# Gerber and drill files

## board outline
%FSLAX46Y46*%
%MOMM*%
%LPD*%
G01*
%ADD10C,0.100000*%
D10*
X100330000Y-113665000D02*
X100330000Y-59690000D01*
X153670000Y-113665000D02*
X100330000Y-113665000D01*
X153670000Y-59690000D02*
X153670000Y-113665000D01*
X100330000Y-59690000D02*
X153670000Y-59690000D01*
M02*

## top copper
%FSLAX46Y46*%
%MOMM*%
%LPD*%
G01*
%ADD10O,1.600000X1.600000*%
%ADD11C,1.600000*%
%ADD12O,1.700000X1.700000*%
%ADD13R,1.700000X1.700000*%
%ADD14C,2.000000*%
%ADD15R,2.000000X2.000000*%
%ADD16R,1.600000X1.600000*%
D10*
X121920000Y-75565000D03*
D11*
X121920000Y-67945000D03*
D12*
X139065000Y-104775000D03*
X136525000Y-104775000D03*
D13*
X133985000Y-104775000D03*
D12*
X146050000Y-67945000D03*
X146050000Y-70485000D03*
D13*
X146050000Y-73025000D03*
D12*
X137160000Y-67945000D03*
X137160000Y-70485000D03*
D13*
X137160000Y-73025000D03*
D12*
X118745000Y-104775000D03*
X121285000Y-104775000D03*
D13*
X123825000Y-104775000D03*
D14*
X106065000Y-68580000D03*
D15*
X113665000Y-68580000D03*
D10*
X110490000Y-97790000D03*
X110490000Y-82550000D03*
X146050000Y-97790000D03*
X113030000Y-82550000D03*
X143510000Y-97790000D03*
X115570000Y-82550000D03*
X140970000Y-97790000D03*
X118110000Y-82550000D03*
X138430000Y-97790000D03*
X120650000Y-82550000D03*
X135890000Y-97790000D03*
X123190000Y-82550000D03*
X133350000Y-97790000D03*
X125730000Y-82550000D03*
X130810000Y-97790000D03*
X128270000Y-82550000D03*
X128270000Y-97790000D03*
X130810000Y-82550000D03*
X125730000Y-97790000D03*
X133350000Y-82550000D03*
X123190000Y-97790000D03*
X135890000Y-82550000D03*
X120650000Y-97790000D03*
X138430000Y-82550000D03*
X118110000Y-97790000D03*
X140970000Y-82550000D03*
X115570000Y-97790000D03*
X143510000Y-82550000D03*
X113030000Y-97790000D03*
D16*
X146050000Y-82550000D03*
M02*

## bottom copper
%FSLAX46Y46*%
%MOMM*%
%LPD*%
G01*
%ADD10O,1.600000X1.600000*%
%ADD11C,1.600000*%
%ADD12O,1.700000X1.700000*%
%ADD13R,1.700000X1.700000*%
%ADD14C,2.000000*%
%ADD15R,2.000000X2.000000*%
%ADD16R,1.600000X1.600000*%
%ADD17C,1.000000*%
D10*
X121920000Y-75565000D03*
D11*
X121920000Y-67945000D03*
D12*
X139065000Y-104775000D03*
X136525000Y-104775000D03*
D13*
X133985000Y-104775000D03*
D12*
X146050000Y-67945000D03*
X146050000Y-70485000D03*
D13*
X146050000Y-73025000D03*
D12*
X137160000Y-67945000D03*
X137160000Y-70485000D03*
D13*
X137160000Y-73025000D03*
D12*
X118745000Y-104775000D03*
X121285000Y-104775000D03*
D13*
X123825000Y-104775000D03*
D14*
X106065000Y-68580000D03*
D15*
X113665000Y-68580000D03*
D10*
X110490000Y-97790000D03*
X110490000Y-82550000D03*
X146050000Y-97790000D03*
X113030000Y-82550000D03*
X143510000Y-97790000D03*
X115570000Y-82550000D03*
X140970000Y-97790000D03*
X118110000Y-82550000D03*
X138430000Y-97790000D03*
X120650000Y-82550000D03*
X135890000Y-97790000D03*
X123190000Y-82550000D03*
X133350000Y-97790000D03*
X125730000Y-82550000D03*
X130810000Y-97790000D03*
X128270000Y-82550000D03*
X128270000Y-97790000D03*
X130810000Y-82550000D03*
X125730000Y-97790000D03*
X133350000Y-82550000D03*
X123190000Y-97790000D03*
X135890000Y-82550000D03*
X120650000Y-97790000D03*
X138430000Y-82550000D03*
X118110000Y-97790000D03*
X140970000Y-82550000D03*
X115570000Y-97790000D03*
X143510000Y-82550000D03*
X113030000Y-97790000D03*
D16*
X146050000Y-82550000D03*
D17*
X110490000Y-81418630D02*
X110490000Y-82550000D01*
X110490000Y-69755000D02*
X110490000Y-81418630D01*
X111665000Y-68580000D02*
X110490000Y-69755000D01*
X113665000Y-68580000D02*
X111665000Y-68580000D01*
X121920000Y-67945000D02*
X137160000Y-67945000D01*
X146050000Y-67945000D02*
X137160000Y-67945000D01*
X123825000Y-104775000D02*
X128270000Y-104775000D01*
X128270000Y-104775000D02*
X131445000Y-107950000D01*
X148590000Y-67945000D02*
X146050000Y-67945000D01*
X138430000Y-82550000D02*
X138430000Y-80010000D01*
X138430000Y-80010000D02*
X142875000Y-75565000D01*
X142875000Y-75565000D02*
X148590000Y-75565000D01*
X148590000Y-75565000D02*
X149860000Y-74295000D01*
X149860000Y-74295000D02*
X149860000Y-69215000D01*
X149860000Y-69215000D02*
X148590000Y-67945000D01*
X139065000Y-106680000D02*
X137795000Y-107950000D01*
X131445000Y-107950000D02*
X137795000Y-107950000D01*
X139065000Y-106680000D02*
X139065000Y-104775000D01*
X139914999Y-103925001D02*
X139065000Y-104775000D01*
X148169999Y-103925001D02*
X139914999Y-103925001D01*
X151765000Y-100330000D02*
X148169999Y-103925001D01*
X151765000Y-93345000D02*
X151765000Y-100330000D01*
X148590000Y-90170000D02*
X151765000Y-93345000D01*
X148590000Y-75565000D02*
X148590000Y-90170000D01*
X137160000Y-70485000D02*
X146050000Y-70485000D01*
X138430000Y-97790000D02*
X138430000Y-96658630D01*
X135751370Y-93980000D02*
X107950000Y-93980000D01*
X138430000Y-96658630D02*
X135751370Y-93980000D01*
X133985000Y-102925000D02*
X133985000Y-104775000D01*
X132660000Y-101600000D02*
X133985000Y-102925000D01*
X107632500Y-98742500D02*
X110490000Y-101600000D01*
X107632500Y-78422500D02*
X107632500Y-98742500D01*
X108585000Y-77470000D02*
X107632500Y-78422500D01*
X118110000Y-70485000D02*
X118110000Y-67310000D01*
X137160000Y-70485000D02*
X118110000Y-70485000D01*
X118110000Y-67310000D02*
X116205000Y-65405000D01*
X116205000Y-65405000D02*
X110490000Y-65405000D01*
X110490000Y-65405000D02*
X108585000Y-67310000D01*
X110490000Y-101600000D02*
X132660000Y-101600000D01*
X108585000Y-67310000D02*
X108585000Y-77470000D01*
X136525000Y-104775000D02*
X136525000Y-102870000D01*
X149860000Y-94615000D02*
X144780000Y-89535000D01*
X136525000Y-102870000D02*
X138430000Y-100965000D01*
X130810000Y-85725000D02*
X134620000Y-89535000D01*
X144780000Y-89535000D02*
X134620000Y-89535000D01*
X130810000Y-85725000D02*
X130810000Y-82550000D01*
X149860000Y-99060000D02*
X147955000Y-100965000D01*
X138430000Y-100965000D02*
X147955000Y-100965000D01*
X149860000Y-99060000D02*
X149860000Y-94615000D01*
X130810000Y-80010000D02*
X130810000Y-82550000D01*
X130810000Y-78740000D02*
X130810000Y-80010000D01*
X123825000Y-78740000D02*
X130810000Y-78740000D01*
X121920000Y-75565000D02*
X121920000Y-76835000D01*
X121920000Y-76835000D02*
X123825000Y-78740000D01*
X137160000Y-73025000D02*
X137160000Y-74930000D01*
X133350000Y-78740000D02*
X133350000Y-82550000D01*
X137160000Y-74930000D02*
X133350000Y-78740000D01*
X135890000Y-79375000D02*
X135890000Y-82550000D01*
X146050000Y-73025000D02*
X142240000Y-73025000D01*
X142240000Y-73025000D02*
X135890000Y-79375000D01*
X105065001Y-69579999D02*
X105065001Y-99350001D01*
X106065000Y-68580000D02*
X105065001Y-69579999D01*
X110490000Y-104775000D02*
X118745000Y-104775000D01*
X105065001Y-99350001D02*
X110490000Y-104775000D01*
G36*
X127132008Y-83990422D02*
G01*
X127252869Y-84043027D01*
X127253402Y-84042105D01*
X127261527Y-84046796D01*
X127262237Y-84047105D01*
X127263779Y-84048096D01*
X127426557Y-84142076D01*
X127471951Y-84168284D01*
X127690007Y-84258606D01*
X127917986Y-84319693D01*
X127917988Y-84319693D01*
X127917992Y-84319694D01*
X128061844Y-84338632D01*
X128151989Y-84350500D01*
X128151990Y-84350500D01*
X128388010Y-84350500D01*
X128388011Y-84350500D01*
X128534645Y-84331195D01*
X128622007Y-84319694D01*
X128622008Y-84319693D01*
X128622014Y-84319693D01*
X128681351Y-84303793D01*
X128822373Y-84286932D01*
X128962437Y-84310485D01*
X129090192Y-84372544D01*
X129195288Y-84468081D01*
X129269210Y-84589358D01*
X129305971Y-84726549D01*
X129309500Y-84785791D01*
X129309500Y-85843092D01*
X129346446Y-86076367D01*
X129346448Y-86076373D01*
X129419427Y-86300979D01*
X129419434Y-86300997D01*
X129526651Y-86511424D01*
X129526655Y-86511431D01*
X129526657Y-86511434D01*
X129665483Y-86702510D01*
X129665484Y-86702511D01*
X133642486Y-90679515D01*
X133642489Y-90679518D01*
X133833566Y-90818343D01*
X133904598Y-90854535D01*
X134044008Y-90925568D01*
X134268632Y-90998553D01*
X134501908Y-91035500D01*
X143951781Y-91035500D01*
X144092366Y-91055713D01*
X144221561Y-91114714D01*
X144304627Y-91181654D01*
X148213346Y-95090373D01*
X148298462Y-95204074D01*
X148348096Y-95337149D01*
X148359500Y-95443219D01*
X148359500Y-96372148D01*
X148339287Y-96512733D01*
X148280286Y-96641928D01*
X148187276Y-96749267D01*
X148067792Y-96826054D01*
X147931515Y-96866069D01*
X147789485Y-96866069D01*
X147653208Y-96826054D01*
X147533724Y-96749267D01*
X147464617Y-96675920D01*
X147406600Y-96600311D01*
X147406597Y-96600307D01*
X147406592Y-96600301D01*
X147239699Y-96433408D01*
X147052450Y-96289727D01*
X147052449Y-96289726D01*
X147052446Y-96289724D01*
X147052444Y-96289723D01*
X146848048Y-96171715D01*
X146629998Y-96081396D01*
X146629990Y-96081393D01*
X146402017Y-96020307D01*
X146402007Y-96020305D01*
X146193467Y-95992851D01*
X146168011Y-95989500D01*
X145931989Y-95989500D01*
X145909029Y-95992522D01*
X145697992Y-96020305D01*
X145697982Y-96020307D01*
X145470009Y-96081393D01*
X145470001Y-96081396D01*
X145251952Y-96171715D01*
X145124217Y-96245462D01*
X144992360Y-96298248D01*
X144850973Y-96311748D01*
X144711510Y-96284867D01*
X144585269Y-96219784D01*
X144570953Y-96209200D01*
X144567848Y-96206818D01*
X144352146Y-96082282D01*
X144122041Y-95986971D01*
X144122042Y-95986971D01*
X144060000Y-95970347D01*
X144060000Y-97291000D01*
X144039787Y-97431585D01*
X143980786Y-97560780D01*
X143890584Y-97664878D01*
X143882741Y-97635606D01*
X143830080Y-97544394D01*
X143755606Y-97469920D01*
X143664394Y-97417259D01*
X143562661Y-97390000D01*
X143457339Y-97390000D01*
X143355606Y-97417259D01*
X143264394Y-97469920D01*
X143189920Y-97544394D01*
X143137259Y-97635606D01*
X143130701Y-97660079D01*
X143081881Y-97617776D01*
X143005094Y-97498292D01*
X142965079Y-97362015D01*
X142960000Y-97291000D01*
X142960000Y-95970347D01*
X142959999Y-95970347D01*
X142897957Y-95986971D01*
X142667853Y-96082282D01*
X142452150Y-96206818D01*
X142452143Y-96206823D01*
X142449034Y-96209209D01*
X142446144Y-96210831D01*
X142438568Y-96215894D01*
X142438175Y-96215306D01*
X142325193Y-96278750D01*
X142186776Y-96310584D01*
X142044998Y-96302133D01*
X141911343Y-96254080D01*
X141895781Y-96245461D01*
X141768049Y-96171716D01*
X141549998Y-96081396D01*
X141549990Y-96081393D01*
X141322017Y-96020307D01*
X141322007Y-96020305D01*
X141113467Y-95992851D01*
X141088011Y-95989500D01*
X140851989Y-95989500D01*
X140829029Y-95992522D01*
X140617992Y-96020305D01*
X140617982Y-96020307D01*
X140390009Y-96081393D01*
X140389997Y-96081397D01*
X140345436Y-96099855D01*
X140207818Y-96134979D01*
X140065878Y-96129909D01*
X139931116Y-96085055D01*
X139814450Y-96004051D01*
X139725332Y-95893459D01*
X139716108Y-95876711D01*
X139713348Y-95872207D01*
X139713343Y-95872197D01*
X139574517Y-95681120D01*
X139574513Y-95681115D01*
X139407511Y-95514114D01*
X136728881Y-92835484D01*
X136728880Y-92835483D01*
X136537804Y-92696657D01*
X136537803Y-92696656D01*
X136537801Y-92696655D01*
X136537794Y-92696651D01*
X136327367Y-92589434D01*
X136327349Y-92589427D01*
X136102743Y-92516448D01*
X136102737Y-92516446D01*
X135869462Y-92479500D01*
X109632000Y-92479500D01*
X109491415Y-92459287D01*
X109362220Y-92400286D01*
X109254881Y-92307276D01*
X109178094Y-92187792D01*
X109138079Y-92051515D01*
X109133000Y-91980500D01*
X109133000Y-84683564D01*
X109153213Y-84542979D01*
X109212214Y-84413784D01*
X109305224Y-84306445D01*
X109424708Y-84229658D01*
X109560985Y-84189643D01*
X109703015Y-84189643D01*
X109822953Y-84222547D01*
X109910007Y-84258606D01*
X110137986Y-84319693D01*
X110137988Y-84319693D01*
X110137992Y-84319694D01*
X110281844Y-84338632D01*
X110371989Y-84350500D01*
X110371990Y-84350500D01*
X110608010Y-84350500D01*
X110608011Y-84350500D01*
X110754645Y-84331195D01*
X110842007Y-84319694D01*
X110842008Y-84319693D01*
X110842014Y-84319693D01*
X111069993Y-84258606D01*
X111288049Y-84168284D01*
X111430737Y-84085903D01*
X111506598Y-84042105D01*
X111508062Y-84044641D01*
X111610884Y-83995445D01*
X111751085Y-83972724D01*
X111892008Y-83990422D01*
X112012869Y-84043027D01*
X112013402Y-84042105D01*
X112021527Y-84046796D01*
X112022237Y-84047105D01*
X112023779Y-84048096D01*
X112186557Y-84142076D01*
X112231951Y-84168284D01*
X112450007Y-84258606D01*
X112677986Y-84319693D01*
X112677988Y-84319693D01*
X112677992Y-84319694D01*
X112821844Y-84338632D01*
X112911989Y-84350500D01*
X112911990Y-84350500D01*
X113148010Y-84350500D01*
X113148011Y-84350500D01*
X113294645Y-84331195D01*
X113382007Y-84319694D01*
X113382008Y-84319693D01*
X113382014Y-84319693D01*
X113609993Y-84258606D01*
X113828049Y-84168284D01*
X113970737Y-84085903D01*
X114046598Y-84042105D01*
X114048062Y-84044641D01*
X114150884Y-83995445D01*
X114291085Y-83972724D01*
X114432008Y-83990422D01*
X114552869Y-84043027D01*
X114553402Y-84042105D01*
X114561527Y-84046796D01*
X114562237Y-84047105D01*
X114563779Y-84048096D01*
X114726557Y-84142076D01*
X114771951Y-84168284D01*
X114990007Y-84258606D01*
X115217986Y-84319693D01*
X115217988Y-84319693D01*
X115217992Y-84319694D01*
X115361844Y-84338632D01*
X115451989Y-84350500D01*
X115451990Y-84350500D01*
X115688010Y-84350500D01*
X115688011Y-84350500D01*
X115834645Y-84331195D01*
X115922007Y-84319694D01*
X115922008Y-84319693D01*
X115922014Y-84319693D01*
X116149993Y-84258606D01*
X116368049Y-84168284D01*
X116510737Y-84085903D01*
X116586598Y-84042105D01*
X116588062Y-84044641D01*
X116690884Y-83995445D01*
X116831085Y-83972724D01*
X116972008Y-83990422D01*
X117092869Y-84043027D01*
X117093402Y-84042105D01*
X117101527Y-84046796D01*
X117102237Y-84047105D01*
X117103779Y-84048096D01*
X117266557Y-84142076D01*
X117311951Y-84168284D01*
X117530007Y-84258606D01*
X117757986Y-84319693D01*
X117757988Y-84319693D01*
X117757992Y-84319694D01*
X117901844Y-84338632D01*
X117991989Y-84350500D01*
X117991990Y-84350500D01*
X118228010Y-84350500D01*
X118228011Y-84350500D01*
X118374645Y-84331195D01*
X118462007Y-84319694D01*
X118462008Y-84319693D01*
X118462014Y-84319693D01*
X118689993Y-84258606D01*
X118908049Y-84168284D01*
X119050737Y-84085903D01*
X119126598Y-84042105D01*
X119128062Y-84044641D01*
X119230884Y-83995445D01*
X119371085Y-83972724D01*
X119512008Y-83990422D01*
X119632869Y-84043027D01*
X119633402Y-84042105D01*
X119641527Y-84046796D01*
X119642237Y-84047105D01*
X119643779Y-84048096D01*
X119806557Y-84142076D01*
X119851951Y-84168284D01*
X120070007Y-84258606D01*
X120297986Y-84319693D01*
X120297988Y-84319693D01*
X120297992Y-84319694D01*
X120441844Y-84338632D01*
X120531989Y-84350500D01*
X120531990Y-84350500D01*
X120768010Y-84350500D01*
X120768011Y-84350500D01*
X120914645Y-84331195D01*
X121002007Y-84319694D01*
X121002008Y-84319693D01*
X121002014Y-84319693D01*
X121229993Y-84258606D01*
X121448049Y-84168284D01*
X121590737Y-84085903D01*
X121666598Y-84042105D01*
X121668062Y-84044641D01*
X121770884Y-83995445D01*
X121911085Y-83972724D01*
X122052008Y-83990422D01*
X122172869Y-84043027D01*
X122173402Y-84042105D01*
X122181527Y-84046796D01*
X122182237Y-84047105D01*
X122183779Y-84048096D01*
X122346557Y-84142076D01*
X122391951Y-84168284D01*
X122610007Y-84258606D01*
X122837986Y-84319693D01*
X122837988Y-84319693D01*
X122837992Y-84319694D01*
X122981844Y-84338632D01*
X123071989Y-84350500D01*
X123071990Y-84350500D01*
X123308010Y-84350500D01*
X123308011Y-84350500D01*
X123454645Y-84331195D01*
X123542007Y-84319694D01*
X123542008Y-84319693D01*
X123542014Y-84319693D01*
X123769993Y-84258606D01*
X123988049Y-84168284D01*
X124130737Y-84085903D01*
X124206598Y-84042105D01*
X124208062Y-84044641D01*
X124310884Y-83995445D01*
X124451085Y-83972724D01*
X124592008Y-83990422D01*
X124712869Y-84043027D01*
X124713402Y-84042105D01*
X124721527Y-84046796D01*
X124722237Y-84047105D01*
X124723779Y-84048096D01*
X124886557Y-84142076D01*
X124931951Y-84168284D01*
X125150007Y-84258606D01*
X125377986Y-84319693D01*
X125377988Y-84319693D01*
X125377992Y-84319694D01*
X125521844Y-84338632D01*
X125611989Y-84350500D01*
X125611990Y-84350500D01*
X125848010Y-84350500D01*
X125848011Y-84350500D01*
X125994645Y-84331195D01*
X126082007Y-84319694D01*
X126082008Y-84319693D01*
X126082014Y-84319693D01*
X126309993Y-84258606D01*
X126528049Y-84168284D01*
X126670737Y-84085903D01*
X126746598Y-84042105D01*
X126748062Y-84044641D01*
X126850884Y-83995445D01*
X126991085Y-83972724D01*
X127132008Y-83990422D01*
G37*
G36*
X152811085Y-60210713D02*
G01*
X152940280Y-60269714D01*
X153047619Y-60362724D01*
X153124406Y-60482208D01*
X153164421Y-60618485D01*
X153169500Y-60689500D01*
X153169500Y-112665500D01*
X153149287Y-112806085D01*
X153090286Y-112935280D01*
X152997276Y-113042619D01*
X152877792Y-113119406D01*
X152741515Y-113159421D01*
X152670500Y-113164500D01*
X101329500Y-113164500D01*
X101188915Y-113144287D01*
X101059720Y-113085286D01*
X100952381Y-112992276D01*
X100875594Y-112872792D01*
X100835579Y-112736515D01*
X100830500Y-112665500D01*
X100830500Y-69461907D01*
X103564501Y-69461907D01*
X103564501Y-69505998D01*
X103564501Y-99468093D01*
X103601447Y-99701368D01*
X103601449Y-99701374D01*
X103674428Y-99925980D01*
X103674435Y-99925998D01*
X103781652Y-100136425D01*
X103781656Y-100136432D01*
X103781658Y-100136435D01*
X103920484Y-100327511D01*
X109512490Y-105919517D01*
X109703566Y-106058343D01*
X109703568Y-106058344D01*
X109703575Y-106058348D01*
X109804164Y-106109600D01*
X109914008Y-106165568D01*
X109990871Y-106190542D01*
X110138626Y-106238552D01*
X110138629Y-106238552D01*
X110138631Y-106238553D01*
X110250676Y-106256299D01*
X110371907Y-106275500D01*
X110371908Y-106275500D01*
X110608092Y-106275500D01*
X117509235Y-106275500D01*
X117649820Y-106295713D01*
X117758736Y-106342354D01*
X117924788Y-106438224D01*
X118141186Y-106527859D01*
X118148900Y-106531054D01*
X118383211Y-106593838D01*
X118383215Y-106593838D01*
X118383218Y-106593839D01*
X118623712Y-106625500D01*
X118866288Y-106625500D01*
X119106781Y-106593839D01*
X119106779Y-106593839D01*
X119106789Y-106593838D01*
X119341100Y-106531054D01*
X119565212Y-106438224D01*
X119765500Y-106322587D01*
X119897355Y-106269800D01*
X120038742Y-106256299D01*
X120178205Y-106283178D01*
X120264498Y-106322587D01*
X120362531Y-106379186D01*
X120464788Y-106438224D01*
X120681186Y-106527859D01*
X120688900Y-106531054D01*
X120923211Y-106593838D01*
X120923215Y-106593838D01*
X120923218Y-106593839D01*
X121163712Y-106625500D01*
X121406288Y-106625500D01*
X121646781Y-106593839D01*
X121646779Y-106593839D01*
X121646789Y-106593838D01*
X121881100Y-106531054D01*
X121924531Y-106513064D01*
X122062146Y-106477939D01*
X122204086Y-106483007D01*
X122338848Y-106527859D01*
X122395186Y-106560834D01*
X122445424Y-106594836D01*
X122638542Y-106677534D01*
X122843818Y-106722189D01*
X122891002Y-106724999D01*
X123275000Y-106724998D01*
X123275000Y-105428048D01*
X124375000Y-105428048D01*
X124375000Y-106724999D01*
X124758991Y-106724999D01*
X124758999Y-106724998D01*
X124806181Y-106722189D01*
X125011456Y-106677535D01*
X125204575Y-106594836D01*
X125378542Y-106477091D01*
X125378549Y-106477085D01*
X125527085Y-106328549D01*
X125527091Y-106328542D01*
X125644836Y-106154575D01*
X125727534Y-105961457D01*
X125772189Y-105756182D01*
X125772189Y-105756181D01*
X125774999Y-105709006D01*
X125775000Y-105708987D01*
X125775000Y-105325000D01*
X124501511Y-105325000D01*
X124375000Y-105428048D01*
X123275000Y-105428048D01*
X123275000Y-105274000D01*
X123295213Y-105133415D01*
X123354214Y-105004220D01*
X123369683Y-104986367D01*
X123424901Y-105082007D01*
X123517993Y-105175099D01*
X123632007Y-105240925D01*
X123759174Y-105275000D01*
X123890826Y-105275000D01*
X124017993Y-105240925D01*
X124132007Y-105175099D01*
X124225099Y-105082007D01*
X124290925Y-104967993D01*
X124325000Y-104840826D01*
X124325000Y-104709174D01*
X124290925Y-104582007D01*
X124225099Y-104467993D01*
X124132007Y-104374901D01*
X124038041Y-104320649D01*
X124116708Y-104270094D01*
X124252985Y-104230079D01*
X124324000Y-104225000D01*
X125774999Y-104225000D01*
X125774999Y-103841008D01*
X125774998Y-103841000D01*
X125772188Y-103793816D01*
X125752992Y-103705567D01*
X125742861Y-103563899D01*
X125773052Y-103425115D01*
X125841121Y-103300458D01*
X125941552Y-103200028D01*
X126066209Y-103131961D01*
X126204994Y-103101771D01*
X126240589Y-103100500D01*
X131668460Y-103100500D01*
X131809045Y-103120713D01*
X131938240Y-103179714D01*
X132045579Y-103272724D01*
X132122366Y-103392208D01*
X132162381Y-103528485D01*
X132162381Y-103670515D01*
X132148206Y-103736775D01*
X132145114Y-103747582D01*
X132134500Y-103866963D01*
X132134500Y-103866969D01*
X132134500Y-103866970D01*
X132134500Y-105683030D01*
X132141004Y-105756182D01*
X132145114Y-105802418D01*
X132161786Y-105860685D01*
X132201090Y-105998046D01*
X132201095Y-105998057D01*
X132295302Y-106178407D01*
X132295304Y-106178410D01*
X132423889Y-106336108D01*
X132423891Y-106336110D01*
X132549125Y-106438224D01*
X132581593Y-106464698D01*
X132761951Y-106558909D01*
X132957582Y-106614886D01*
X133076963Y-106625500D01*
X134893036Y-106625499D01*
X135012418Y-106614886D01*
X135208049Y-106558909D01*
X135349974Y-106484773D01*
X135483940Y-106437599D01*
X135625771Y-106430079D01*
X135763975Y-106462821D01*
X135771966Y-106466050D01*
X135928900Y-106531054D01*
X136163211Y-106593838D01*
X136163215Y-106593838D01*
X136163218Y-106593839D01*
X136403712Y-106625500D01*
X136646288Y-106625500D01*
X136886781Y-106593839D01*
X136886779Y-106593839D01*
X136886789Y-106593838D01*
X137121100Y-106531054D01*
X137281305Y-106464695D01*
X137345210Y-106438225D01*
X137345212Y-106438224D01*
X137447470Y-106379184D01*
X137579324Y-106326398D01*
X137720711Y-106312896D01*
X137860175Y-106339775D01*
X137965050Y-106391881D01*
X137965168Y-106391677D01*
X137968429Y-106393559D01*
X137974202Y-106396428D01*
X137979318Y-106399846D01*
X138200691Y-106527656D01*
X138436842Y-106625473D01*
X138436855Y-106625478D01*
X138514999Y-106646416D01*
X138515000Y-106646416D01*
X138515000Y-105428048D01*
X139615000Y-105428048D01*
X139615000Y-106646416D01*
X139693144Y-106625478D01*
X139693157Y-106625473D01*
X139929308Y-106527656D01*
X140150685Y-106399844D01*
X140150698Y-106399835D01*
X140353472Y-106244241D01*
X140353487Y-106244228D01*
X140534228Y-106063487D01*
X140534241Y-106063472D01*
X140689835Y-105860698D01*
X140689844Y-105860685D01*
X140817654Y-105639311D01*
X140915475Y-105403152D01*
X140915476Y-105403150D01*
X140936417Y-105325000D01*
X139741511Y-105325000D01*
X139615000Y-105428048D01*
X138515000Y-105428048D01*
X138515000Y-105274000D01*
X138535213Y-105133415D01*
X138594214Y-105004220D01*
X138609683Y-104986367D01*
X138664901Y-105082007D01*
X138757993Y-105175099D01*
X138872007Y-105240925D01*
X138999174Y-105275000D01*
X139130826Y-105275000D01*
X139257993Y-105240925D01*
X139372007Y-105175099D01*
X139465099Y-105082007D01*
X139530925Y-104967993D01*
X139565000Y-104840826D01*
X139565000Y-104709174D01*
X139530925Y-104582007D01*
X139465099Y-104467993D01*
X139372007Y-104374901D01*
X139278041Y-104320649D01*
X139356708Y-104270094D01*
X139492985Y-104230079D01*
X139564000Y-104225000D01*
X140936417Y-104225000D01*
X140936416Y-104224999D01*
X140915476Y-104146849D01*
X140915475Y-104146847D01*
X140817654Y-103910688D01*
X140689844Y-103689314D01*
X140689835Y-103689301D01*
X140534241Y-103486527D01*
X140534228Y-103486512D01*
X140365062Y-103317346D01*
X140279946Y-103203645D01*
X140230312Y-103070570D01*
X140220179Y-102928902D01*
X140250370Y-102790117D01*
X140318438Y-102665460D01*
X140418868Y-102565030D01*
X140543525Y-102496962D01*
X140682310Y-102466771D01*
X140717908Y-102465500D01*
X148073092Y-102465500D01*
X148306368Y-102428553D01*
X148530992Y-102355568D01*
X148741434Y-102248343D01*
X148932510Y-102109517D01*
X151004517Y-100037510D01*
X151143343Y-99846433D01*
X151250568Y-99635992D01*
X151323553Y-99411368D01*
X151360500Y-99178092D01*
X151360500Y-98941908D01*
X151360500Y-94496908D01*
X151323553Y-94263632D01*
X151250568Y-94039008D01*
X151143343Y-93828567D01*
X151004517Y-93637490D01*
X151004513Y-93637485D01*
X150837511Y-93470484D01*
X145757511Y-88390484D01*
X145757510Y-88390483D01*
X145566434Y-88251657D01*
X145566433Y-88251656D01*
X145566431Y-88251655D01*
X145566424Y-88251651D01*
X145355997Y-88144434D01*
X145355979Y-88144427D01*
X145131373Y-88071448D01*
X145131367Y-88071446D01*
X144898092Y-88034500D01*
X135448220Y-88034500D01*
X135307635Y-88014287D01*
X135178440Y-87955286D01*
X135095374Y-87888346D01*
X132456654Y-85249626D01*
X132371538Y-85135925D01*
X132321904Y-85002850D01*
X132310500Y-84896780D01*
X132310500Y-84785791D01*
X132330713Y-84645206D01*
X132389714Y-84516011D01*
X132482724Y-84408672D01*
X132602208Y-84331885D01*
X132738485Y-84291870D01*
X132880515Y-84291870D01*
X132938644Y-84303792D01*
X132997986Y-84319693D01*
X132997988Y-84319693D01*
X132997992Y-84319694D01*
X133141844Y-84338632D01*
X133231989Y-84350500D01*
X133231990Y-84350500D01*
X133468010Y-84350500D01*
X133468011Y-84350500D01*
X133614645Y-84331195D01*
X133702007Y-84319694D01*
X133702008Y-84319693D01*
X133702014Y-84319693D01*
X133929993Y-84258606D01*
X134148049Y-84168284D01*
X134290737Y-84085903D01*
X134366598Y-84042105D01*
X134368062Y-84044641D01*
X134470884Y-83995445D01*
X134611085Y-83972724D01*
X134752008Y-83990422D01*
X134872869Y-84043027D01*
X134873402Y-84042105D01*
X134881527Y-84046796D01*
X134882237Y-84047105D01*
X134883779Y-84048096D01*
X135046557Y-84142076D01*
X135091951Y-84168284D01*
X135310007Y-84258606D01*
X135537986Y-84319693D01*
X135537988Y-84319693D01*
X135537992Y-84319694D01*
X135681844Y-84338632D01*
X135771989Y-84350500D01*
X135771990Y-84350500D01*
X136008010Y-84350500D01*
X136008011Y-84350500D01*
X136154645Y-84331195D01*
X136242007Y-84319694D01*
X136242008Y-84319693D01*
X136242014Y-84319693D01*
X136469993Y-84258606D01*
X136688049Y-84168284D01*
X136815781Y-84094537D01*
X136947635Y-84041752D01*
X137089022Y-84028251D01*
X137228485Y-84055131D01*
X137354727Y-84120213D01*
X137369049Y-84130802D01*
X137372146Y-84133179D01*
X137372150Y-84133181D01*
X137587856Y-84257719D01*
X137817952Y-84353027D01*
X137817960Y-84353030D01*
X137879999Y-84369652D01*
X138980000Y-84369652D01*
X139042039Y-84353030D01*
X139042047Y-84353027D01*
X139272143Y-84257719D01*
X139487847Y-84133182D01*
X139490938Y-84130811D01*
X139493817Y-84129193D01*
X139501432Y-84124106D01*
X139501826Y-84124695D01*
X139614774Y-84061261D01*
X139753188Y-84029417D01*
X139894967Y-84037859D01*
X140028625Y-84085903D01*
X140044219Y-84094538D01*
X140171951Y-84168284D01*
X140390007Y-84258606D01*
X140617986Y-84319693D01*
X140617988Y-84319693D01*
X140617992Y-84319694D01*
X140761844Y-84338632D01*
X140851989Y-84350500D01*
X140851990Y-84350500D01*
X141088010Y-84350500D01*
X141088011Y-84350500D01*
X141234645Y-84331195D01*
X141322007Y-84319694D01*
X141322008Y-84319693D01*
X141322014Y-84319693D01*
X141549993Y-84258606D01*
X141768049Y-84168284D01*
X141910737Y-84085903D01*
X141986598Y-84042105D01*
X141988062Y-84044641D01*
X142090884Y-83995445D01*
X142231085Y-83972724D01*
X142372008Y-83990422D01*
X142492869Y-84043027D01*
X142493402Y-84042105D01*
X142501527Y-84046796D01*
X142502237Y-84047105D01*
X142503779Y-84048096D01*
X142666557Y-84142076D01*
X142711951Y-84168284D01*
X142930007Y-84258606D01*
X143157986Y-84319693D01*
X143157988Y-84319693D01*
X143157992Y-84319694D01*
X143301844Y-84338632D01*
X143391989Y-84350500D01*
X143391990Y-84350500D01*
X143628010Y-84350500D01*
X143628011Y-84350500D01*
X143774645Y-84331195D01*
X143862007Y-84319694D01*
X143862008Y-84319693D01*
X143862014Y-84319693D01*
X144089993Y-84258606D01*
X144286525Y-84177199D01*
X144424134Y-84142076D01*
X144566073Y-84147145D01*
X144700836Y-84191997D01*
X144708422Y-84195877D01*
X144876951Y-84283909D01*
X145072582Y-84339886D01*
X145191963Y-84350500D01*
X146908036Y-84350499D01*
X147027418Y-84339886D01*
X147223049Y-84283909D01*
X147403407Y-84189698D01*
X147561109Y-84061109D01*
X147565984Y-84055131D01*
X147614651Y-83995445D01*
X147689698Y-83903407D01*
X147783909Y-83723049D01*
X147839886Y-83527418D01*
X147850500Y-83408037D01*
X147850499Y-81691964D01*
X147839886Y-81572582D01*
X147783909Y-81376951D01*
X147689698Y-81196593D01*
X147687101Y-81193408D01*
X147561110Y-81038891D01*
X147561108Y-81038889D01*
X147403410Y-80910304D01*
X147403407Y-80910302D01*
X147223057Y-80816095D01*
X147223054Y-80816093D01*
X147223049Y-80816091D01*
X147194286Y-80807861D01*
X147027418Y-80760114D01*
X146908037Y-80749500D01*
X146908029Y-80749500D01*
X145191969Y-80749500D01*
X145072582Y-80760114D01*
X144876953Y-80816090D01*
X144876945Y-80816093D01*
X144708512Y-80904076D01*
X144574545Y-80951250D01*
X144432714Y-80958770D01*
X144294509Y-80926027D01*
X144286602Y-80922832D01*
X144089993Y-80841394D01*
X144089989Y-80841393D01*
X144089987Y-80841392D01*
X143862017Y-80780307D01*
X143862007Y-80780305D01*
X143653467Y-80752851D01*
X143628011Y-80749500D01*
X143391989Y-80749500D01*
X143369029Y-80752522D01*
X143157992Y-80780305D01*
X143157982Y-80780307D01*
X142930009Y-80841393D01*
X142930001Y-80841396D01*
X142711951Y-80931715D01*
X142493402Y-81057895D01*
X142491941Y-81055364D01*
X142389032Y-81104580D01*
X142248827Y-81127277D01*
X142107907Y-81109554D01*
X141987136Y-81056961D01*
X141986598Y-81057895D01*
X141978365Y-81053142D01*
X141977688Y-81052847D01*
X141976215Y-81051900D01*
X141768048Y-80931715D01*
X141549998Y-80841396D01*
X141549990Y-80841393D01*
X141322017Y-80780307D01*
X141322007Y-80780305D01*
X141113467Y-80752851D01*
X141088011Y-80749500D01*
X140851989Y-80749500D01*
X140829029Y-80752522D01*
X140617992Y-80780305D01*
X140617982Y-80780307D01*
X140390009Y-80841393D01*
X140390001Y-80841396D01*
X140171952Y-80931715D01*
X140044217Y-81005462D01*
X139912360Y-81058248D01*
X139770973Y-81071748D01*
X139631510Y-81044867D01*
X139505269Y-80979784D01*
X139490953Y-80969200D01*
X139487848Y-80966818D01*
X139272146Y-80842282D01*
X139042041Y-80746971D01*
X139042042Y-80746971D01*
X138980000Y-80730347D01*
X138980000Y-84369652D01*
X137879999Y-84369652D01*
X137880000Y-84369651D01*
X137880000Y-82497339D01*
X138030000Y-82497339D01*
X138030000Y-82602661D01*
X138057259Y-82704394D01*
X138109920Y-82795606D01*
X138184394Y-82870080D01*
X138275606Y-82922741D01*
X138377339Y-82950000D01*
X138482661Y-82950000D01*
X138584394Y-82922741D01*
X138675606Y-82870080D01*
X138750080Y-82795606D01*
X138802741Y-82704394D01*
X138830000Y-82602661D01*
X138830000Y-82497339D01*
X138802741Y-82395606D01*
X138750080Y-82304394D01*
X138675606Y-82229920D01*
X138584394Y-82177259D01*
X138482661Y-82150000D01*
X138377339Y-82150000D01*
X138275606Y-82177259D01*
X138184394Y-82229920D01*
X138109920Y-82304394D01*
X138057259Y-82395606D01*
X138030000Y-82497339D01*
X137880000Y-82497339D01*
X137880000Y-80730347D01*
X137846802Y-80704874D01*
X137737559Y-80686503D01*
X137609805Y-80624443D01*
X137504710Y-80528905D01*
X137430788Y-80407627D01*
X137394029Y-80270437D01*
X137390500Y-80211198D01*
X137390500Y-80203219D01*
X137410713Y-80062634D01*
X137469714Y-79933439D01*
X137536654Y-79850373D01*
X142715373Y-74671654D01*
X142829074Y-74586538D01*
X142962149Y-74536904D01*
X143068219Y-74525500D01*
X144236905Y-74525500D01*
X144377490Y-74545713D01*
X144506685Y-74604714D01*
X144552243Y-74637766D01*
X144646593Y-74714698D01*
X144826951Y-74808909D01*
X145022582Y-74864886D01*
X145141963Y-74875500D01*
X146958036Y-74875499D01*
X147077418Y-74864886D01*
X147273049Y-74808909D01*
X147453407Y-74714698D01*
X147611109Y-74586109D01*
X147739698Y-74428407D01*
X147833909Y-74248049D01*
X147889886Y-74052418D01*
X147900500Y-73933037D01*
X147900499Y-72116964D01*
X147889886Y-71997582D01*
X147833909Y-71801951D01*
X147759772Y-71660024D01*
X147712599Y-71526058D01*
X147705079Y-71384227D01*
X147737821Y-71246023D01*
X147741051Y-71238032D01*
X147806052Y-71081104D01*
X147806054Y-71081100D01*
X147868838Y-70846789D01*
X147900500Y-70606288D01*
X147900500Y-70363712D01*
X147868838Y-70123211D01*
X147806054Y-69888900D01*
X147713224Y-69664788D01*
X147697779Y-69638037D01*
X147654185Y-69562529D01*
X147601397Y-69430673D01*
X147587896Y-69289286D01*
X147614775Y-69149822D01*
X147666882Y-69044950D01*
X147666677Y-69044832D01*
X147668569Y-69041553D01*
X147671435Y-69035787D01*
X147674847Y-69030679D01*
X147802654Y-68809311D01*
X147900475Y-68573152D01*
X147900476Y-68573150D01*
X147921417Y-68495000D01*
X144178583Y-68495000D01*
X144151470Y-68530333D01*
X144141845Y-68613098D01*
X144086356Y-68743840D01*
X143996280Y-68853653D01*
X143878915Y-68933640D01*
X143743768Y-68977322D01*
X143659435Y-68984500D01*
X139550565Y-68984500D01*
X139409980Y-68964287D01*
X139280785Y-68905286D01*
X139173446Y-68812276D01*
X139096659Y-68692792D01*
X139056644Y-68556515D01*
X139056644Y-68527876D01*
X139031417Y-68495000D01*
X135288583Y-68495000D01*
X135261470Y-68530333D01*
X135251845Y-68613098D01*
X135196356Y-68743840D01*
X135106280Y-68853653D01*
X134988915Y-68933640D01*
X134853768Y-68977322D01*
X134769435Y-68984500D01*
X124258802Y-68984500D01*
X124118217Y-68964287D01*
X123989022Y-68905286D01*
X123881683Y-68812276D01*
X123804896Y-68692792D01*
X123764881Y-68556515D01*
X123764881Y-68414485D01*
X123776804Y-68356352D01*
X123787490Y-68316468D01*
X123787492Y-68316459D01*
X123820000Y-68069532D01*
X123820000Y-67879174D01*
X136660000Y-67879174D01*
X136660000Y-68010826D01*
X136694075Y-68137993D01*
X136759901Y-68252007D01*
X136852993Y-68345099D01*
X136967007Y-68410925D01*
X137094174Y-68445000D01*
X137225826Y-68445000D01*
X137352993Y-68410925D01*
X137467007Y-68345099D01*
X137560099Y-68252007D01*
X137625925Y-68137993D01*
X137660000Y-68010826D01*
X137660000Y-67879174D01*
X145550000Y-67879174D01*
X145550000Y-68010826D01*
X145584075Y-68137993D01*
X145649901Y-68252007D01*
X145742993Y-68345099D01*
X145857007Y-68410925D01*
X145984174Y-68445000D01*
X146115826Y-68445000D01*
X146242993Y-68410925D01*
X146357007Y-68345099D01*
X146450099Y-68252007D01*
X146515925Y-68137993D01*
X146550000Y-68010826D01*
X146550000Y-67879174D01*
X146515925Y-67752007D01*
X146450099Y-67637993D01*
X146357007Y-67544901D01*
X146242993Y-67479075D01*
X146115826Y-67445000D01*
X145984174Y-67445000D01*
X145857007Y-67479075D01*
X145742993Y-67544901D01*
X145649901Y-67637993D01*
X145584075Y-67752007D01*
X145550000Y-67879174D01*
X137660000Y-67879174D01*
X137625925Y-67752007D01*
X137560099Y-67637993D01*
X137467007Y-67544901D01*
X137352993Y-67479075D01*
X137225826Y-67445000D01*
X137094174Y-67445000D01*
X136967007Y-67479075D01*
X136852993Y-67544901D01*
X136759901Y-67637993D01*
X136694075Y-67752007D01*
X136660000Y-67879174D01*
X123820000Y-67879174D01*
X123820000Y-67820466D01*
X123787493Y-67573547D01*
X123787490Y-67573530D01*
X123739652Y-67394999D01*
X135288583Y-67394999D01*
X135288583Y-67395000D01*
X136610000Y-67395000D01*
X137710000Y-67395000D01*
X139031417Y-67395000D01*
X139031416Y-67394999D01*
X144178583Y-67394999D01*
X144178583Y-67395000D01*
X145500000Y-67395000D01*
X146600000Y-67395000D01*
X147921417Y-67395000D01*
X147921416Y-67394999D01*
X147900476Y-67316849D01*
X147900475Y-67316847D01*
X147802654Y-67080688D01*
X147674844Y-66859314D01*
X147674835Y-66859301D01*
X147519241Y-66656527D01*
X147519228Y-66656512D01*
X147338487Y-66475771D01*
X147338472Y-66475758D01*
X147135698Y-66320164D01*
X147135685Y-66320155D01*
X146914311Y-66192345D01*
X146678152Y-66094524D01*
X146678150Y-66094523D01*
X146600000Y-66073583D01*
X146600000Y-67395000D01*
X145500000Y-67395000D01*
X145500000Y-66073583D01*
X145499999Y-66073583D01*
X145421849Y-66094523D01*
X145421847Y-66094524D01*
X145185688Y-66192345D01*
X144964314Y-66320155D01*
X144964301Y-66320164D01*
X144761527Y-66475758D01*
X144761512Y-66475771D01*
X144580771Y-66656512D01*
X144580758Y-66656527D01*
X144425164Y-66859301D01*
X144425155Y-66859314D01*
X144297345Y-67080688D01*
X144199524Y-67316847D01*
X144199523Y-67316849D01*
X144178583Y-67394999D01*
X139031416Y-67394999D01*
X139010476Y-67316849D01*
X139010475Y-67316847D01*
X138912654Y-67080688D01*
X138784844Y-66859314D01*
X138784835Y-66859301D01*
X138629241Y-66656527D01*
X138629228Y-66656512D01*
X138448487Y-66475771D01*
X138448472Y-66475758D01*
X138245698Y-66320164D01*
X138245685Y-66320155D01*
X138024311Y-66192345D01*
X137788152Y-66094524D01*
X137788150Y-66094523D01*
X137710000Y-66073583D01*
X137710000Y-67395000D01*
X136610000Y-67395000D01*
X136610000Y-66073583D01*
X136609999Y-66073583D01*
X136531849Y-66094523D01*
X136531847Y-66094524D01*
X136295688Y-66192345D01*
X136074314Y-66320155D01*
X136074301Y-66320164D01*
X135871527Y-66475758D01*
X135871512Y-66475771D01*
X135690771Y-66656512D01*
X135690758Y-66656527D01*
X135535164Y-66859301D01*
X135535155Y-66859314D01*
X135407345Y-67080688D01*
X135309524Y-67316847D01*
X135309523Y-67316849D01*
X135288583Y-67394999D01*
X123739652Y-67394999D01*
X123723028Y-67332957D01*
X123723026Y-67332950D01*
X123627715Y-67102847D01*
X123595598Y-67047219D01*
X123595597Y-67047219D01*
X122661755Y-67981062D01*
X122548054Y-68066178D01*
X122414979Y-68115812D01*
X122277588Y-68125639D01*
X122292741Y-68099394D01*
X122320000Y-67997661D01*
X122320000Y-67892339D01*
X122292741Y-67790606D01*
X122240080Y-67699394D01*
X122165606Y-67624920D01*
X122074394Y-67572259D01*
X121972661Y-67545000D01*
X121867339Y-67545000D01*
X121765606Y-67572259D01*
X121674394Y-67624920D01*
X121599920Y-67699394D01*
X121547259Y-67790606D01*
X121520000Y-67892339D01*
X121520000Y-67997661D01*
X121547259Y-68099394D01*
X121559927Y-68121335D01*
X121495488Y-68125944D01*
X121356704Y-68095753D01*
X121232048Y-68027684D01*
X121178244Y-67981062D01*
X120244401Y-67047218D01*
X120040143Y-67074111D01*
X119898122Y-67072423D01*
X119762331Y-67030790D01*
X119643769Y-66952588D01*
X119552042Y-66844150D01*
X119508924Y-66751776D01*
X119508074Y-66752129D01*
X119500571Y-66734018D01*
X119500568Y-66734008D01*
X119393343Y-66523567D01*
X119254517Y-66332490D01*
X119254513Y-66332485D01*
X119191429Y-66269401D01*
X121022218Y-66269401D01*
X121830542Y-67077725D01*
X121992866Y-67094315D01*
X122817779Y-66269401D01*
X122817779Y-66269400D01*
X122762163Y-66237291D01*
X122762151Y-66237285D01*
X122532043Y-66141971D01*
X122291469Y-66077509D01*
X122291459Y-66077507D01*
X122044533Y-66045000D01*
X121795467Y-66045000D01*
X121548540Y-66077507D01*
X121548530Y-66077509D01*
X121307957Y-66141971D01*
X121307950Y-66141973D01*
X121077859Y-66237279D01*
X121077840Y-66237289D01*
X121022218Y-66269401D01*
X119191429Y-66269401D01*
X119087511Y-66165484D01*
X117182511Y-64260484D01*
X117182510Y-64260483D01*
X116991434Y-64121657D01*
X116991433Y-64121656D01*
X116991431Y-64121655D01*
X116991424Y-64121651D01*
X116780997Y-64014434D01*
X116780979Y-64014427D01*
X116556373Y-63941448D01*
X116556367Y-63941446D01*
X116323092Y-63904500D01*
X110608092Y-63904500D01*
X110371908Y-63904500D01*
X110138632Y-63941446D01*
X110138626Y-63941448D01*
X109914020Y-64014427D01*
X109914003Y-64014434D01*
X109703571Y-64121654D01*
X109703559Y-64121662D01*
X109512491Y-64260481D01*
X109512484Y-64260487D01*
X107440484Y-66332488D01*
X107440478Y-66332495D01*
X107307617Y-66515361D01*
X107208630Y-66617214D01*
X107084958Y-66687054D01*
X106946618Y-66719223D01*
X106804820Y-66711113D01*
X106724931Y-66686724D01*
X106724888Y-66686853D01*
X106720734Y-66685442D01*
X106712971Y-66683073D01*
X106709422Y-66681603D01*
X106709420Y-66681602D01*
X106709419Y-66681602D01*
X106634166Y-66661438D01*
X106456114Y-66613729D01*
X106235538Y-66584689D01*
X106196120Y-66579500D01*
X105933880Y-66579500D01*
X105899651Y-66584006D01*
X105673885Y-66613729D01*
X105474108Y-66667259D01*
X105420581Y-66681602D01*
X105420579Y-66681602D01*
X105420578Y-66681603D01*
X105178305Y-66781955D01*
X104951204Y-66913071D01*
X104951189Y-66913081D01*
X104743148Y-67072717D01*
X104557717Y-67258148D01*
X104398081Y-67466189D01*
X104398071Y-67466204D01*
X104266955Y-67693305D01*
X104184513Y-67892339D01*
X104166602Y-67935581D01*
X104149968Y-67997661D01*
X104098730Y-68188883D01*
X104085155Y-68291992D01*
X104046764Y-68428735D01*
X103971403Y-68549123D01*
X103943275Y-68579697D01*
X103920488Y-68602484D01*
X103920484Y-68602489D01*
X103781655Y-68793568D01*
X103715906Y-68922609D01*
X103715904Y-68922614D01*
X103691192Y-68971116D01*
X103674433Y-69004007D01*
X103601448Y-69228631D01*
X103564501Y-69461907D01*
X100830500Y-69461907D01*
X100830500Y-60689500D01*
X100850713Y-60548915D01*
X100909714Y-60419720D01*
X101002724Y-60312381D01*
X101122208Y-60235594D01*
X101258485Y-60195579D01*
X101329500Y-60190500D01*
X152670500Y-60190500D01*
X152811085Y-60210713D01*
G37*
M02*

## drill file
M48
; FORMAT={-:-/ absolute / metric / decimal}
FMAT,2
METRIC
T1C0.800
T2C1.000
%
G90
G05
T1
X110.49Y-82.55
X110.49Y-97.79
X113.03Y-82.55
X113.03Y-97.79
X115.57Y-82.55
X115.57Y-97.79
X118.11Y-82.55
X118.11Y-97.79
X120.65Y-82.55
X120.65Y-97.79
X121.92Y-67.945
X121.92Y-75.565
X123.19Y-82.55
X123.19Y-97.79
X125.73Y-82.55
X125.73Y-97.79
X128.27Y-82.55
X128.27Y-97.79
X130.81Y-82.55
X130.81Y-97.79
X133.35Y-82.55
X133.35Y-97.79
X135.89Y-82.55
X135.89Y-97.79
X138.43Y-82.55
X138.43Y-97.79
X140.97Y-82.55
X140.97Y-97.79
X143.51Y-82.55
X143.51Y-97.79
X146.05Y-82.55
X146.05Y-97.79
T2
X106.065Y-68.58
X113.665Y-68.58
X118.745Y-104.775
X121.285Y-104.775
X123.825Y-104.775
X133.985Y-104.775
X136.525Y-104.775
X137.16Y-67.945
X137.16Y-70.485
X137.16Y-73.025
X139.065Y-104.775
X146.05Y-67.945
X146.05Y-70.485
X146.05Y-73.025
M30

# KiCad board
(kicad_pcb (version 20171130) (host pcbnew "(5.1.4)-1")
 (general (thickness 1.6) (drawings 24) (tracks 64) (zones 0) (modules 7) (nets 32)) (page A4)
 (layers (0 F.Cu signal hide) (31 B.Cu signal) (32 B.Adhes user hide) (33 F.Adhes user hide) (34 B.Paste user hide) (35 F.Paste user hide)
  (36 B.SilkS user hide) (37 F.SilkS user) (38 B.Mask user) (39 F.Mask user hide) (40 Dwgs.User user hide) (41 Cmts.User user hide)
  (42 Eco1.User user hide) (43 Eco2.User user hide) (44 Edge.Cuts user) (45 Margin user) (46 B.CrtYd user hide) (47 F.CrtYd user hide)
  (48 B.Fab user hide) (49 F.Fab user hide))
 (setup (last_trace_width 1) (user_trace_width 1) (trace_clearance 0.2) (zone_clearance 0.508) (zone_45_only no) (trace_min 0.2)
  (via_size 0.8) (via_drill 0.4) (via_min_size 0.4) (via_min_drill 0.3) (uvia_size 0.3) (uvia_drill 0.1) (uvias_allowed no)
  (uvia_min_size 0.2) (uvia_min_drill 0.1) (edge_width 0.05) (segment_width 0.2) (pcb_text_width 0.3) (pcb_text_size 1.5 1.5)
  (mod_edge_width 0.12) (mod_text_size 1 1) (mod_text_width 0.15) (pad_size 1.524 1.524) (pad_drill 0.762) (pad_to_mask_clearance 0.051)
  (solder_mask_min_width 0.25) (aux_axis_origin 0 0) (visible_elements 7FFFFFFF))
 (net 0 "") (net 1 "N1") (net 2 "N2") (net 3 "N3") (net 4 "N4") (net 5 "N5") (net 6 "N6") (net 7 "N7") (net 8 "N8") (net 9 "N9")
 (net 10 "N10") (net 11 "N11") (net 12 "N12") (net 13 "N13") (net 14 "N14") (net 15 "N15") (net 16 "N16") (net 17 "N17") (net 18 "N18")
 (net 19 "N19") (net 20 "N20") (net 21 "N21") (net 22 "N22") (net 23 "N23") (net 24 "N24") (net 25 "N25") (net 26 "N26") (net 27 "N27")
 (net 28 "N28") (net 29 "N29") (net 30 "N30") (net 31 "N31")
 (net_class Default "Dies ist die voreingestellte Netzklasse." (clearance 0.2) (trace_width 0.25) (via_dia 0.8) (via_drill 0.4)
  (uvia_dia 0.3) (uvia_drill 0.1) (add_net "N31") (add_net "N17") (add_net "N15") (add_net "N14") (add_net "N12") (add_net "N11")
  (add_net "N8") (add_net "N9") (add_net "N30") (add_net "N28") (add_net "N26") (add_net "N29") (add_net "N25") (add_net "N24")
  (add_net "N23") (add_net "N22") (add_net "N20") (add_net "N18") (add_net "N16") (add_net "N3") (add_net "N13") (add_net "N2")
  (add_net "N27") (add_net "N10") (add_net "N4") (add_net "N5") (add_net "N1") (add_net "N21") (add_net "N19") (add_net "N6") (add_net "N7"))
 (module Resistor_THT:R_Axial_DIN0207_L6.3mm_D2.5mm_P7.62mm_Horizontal (layer F.Cu) (at 121.92 67.945 270)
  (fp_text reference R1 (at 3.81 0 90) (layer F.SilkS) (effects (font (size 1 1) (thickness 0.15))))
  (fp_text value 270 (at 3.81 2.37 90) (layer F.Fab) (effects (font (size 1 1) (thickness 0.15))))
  (pad 2 thru_hole oval (at 7.62 0 270) (size 1.6 1.6) (drill 0.8) (layers *.Cu *.Mask) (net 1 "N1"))
  (pad 1 thru_hole circle (at 0 0 270) (size 1.6 1.6) (drill 0.8) (layers *.Cu *.Mask) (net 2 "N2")))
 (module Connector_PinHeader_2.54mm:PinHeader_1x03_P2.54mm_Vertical (layer F.Cu) (at 133.985 104.775 90)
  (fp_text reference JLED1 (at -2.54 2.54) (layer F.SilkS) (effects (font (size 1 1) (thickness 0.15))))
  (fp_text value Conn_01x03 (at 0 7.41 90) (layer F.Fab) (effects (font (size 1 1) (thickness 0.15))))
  (pad 3 thru_hole oval (at 0 5.08 90) (size 1.7 1.7) (drill 1) (layers *.Cu *.Mask) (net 2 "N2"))
  (pad 2 thru_hole oval (at 0 2.54 90) (size 1.7 1.7) (drill 1) (layers *.Cu *.Mask) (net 1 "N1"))
  (pad 1 thru_hole rect (at 0 0 90) (size 1.7 1.7) (drill 1) (layers *.Cu *.Mask) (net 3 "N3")))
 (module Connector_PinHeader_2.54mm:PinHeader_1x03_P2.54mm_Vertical (layer F.Cu) (at 146.05 73.025 180)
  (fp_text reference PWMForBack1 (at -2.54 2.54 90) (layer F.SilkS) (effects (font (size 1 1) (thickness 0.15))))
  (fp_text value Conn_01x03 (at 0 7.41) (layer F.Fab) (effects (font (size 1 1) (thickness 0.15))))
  (pad 3 thru_hole oval (at 0 5.08 180) (size 1.7 1.7) (drill 1) (layers *.Cu *.Mask) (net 2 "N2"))
  (pad 2 thru_hole oval (at 0 2.54 180) (size 1.7 1.7) (drill 1) (layers *.Cu *.Mask) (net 3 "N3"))
  (pad 1 thru_hole rect (at 0 0 180) (size 1.7 1.7) (drill 1) (layers *.Cu *.Mask) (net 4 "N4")))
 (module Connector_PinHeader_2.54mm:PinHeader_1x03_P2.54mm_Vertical (layer F.Cu) (at 137.16 73.025 180)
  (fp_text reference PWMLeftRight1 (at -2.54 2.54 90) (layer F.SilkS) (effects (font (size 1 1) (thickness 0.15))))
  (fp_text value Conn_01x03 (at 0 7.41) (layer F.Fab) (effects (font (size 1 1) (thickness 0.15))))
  (pad 3 thru_hole oval (at 0 5.08 180) (size 1.7 1.7) (drill 1) (layers *.Cu *.Mask) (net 2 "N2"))
  (pad 2 thru_hole oval (at 0 2.54 180) (size 1.7 1.7) (drill 1) (layers *.Cu *.Mask) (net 3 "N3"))
  (pad 1 thru_hole rect (at 0 0 180) (size 1.7 1.7) (drill 1) (layers *.Cu *.Mask) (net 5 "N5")))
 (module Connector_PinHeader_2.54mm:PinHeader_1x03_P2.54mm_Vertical (layer F.Cu) (at 123.825 104.775 270)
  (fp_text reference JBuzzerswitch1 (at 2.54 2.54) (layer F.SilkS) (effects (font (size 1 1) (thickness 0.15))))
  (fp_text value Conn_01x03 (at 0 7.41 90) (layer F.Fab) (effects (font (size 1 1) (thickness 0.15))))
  (pad 3 thru_hole oval (at 0 5.08 270) (size 1.7 1.7) (drill 1) (layers *.Cu *.Mask) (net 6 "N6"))
  (pad 2 thru_hole oval (at 0 2.54 270) (size 1.7 1.7) (drill 1) (layers *.Cu *.Mask) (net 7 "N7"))
  (pad 1 thru_hole rect (at 0 0 270) (size 1.7 1.7) (drill 1) (layers *.Cu *.Mask) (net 2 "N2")))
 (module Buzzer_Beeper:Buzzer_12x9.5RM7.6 (layer F.Cu) (at 113.665 68.58 180)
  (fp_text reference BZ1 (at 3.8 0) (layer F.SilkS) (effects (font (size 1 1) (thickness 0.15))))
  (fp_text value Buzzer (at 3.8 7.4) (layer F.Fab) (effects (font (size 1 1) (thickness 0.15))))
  (pad 2 thru_hole circle (at 7.6 0 180) (size 2 2) (drill 1) (layers *.Cu *.Mask) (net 6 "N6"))
  (pad 1 thru_hole rect (at 0 0 180) (size 2 2) (drill 1) (layers *.Cu *.Mask) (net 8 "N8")))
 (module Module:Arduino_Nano (layer F.Cu) (at 146.05 82.55 270)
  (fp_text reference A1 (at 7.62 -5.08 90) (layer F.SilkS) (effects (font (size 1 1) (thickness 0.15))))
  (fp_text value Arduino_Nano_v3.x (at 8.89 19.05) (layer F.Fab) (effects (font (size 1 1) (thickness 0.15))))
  (pad 16 thru_hole oval (at 15.24 35.56 270) (size 1.6 1.6) (drill 0.8) (layers *.Cu *.Mask) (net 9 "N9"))
  (pad 15 thru_hole oval (at 0 35.56 270) (size 1.6 1.6) (drill 0.8) (layers *.Cu *.Mask) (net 8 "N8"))
  (pad 30 thru_hole oval (at 15.24 0 270) (size 1.6 1.6) (drill 0.8) (layers *.Cu *.Mask) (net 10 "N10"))
  (pad 14 thru_hole oval (at 0 33.02 270) (size 1.6 1.6) (drill 0.8) (layers *.Cu *.Mask) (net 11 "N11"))
  (pad 29 thru_hole oval (at 15.24 2.54 270) (size 1.6 1.6) (drill 0.8) (layers *.Cu *.Mask) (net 2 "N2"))
  (pad 13 thru_hole oval (at 0 30.48 270) (size 1.6 1.6) (drill 0.8) (layers *.Cu *.Mask) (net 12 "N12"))
  (pad 28 thru_hole oval (at 15.24 5.08 270) (size 1.6 1.6) (drill 0.8) (layers *.Cu *.Mask) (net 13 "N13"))
  (pad 12 thru_hole oval (at 0 27.94 270) (size 1.6 1.6) (drill 0.8) (layers *.Cu *.Mask) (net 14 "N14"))
  (pad 27 thru_hole oval (at 15.24 7.62 270) (size 1.6 1.6) (drill 0.8) (layers *.Cu *.Mask) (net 3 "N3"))
  (pad 11 thru_hole oval (at 0 25.4 270) (size 1.6 1.6) (drill 0.8) (layers *.Cu *.Mask) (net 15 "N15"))
  (pad 26 thru_hole oval (at 15.24 10.16 270) (size 1.6 1.6) (drill 0.8) (layers *.Cu *.Mask) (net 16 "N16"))
  (pad 10 thru_hole oval (at 0 22.86 270) (size 1.6 1.6) (drill 0.8) (layers *.Cu *.Mask) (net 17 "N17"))
  (pad 25 thru_hole oval (at 15.24 12.7 270) (size 1.6 1.6) (drill 0.8) (layers *.Cu *.Mask) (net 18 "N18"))
  (pad 9 thru_hole oval (at 0 20.32 270) (size 1.6 1.6) (drill 0.8) (layers *.Cu *.Mask) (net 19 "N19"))
  (pad 24 thru_hole oval (at 15.24 15.24 270) (size 1.6 1.6) (drill 0.8) (layers *.Cu *.Mask) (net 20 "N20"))
  (pad 8 thru_hole oval (at 0 17.78 270) (size 1.6 1.6) (drill 0.8) (layers *.Cu *.Mask) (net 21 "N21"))
  (pad 23 thru_hole oval (at 15.24 17.78 270) (size 1.6 1.6) (drill 0.8) (layers *.Cu *.Mask) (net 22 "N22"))
  (pad 7 thru_hole oval (at 0 15.24 270) (size 1.6 1.6) (drill 0.8) (layers *.Cu *.Mask) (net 1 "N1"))
  (pad 22 thru_hole oval (at 15.24 20.32 270) (size 1.6 1.6) (drill 0.8) (layers *.Cu *.Mask) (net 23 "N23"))
  (pad 6 thru_hole oval (at 0 12.7 270) (size 1.6 1.6) (drill 0.8) (layers *.Cu *.Mask) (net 5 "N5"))
  (pad 21 thru_hole oval (at 15.24 22.86 270) (size 1.6 1.6) (drill 0.8) (layers *.Cu *.Mask) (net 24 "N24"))
  (pad 5 thru_hole oval (at 0 10.16 270) (size 1.6 1.6) (drill 0.8) (layers *.Cu *.Mask) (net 4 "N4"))
  (pad 20 thru_hole oval (at 15.24 25.4 270) (size 1.6 1.6) (drill 0.8) (layers *.Cu *.Mask) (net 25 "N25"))
  (pad 4 thru_hole oval (at 0 7.62 270) (size 1.6 1.6) (drill 0.8) (layers *.Cu *.Mask) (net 2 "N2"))
  (pad 19 thru_hole oval (at 15.24 27.94 270) (size 1.6 1.6) (drill 0.8) (layers *.Cu *.Mask) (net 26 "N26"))
  (pad 3 thru_hole oval (at 0 5.08 270) (size 1.6 1.6) (drill 0.8) (layers *.Cu *.Mask) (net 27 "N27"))
  (pad 18 thru_hole oval (at 15.24 30.48 270) (size 1.6 1.6) (drill 0.8) (layers *.Cu *.Mask) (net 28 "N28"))
  (pad 2 thru_hole oval (at 0 2.54 270) (size 1.6 1.6) (drill 0.8) (layers *.Cu *.Mask) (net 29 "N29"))
  (pad 17 thru_hole oval (at 15.24 33.02 270) (size 1.6 1.6) (drill 0.8) (layers *.Cu *.Mask) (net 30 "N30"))
  (pad 1 thru_hole rect (at 0 0 270) (size 1.6 1.6) (drill 0.8) (layers *.Cu *.Mask) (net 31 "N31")))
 (gr_line (start 100.33 113.665) (end 100.33 59.69) (layer Edge.Cuts) (width 0.1))
 (gr_line (start 153.67 113.665) (end 100.33 113.665) (layer Edge.Cuts) (width 0.1))
 (gr_line (start 153.67 59.69) (end 153.67 113.665) (layer Edge.Cuts) (width 0.1))
 (gr_line (start 100.33 59.69) (end 153.67 59.69) (layer Edge.Cuts) (width 0.1))
 (segment (start 110.49 81.41863) (end 110.49 82.55) (width 1) (layer B.Cu) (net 8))
 (segment (start 110.49 69.755) (end 110.49 81.41863) (width 1) (layer B.Cu) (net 8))
 (segment (start 111.665 68.58) (end 110.49 69.755) (width 1) (layer B.Cu) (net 8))
 (segment (start 113.665 68.58) (end 111.665 68.58) (width 1) (layer B.Cu) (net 8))
 (segment (start 121.92 67.945) (end 137.16 67.945) (width 1) (layer B.Cu) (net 2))
 (segment (start 146.05 67.945) (end 137.16 67.945) (width 1) (layer B.Cu) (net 2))
 (segment (start 123.825 104.775) (end 128.27 104.775) (width 1) (layer B.Cu) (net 2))
 (segment (start 128.27 104.775) (end 131.445 107.95) (width 1) (layer B.Cu) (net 2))
 (segment (start 148.59 67.945) (end 146.05 67.945) (width 1) (layer B.Cu) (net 2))
 (segment (start 138.43 82.55) (end 138.43 80.01) (width 1) (layer B.Cu) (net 2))
 (segment (start 138.43 80.01) (end 142.875 75.565) (width 1) (layer B.Cu) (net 2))
 (segment (start 142.875 75.565) (end 148.59 75.565) (width 1) (layer B.Cu) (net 2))
 (segment (start 148.59 75.565) (end 149.86 74.295) (width 1) (layer B.Cu) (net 2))
 (segment (start 149.86 74.295) (end 149.86 69.215) (width 1) (layer B.Cu) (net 2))
 (segment (start 149.86 69.215) (end 148.59 67.945) (width 1) (layer B.Cu) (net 2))
 (segment (start 139.065 106.68) (end 137.795 107.95) (width 1) (layer B.Cu) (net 2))
 (segment (start 131.445 107.95) (end 137.795 107.95) (width 1) (layer B.Cu) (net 2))
 (segment (start 139.065 106.68) (end 139.065 104.775) (width 1) (layer B.Cu) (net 2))
 (segment (start 139.914999 103.925001) (end 139.065 104.775) (width 1) (layer B.Cu) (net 2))
 (segment (start 148.169999 103.925001) (end 139.914999 103.925001) (width 1) (layer B.Cu) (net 2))
 (segment (start 151.765 100.33) (end 148.169999 103.925001) (width 1) (layer B.Cu) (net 2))
 (segment (start 151.765 93.345) (end 151.765 100.33) (width 1) (layer B.Cu) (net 2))
 (segment (start 148.59 90.17) (end 151.765 93.345) (width 1) (layer B.Cu) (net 2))
 (segment (start 148.59 75.565) (end 148.59 90.17) (width 1) (layer B.Cu) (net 2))
 (segment (start 137.16 70.485) (end 146.05 70.485) (width 1) (layer B.Cu) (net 3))
 (segment (start 138.43 97.79) (end 138.43 96.65863) (width 1) (layer B.Cu) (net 3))
 (segment (start 135.75137 93.98) (end 107.95 93.98) (width 1) (layer B.Cu) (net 3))
 (segment (start 138.43 96.65863) (end 135.75137 93.98) (width 1) (layer B.Cu) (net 3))
 (segment (start 133.985 102.925) (end 133.985 104.775) (width 1) (layer B.Cu) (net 3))
 (segment (start 132.66 101.6) (end 133.985 102.925) (width 1) (layer B.Cu) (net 3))
 (segment (start 107.6325 98.7425) (end 110.49 101.6) (width 1) (layer B.Cu) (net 3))
 (segment (start 107.6325 78.4225) (end 107.6325 98.7425) (width 1) (layer B.Cu) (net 3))
 (segment (start 108.585 77.47) (end 107.6325 78.4225) (width 1) (layer B.Cu) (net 3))
 (segment (start 118.11 70.485) (end 118.11 67.31) (width 1) (layer B.Cu) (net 3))
 (segment (start 137.16 70.485) (end 118.11 70.485) (width 1) (layer B.Cu) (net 3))
 (segment (start 118.11 67.31) (end 116.205 65.405) (width 1) (layer B.Cu) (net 3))
 (segment (start 116.205 65.405) (end 110.49 65.405) (width 1) (layer B.Cu) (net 3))
 (segment (start 110.49 65.405) (end 108.585 67.31) (width 1) (layer B.Cu) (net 3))
 (segment (start 110.49 101.6) (end 132.66 101.6) (width 1) (layer B.Cu) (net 3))
 (segment (start 108.585 67.31) (end 108.585 77.47) (width 1) (layer B.Cu) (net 3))
 (segment (start 136.525 104.775) (end 136.525 102.87) (width 1) (layer B.Cu) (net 1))
 (segment (start 149.86 94.615) (end 144.78 89.535) (width 1) (layer B.Cu) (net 1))
 (segment (start 136.525 102.87) (end 138.43 100.965) (width 1) (layer B.Cu) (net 1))
 (segment (start 130.81 85.725) (end 134.62 89.535) (width 1) (layer B.Cu) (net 1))
 (segment (start 144.78 89.535) (end 134.62 89.535) (width 1) (layer B.Cu) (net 1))
 (segment (start 130.81 85.725) (end 130.81 82.55) (width 1) (layer B.Cu) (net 1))
 (segment (start 149.86 99.06) (end 147.955 100.965) (width 1) (layer B.Cu) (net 1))
 (segment (start 138.43 100.965) (end 147.955 100.965) (width 1) (layer B.Cu) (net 1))
 (segment (start 149.86 99.06) (end 149.86 94.615) (width 1) (layer B.Cu) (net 1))
 (segment (start 130.81 80.01) (end 130.81 82.55) (width 1) (layer B.Cu) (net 1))
 (segment (start 130.81 78.74) (end 130.81 80.01) (width 1) (layer B.Cu) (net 1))
 (segment (start 123.825 78.74) (end 130.81 78.74) (width 1) (layer B.Cu) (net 1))
 (segment (start 121.92 75.565) (end 121.92 76.835) (width 1) (layer B.Cu) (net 1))
 (segment (start 121.92 76.835) (end 123.825 78.74) (width 1) (layer B.Cu) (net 1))
 (segment (start 137.16 73.025) (end 137.16 74.93) (width 1) (layer B.Cu) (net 5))
 (segment (start 133.35 78.74) (end 133.35 82.55) (width 1) (layer B.Cu) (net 5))
 (segment (start 137.16 74.93) (end 133.35 78.74) (width 1) (layer B.Cu) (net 5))
 (segment (start 135.89 79.375) (end 135.89 82.55) (width 1) (layer B.Cu) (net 4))
 (segment (start 146.05 73.025) (end 142.24 73.025) (width 1) (layer B.Cu) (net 4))
 (segment (start 142.24 73.025) (end 135.89 79.375) (width 1) (layer B.Cu) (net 4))
 (segment (start 105.065001 69.579999) (end 105.065001 99.350001) (width 1) (layer B.Cu) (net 6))
 (segment (start 106.065 68.58) (end 105.065001 69.579999) (width 1) (layer B.Cu) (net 6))
 (segment (start 110.49 104.775) (end 118.745 104.775) (width 1) (layer B.Cu) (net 6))
 (segment (start 105.065001 99.350001) (end 110.49 104.775) (width 1) (layer B.Cu) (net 6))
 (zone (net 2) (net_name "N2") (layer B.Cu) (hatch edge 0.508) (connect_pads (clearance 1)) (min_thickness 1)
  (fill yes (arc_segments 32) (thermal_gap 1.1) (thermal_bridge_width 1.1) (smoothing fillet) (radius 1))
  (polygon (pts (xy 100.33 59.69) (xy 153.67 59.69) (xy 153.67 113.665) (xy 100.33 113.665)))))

